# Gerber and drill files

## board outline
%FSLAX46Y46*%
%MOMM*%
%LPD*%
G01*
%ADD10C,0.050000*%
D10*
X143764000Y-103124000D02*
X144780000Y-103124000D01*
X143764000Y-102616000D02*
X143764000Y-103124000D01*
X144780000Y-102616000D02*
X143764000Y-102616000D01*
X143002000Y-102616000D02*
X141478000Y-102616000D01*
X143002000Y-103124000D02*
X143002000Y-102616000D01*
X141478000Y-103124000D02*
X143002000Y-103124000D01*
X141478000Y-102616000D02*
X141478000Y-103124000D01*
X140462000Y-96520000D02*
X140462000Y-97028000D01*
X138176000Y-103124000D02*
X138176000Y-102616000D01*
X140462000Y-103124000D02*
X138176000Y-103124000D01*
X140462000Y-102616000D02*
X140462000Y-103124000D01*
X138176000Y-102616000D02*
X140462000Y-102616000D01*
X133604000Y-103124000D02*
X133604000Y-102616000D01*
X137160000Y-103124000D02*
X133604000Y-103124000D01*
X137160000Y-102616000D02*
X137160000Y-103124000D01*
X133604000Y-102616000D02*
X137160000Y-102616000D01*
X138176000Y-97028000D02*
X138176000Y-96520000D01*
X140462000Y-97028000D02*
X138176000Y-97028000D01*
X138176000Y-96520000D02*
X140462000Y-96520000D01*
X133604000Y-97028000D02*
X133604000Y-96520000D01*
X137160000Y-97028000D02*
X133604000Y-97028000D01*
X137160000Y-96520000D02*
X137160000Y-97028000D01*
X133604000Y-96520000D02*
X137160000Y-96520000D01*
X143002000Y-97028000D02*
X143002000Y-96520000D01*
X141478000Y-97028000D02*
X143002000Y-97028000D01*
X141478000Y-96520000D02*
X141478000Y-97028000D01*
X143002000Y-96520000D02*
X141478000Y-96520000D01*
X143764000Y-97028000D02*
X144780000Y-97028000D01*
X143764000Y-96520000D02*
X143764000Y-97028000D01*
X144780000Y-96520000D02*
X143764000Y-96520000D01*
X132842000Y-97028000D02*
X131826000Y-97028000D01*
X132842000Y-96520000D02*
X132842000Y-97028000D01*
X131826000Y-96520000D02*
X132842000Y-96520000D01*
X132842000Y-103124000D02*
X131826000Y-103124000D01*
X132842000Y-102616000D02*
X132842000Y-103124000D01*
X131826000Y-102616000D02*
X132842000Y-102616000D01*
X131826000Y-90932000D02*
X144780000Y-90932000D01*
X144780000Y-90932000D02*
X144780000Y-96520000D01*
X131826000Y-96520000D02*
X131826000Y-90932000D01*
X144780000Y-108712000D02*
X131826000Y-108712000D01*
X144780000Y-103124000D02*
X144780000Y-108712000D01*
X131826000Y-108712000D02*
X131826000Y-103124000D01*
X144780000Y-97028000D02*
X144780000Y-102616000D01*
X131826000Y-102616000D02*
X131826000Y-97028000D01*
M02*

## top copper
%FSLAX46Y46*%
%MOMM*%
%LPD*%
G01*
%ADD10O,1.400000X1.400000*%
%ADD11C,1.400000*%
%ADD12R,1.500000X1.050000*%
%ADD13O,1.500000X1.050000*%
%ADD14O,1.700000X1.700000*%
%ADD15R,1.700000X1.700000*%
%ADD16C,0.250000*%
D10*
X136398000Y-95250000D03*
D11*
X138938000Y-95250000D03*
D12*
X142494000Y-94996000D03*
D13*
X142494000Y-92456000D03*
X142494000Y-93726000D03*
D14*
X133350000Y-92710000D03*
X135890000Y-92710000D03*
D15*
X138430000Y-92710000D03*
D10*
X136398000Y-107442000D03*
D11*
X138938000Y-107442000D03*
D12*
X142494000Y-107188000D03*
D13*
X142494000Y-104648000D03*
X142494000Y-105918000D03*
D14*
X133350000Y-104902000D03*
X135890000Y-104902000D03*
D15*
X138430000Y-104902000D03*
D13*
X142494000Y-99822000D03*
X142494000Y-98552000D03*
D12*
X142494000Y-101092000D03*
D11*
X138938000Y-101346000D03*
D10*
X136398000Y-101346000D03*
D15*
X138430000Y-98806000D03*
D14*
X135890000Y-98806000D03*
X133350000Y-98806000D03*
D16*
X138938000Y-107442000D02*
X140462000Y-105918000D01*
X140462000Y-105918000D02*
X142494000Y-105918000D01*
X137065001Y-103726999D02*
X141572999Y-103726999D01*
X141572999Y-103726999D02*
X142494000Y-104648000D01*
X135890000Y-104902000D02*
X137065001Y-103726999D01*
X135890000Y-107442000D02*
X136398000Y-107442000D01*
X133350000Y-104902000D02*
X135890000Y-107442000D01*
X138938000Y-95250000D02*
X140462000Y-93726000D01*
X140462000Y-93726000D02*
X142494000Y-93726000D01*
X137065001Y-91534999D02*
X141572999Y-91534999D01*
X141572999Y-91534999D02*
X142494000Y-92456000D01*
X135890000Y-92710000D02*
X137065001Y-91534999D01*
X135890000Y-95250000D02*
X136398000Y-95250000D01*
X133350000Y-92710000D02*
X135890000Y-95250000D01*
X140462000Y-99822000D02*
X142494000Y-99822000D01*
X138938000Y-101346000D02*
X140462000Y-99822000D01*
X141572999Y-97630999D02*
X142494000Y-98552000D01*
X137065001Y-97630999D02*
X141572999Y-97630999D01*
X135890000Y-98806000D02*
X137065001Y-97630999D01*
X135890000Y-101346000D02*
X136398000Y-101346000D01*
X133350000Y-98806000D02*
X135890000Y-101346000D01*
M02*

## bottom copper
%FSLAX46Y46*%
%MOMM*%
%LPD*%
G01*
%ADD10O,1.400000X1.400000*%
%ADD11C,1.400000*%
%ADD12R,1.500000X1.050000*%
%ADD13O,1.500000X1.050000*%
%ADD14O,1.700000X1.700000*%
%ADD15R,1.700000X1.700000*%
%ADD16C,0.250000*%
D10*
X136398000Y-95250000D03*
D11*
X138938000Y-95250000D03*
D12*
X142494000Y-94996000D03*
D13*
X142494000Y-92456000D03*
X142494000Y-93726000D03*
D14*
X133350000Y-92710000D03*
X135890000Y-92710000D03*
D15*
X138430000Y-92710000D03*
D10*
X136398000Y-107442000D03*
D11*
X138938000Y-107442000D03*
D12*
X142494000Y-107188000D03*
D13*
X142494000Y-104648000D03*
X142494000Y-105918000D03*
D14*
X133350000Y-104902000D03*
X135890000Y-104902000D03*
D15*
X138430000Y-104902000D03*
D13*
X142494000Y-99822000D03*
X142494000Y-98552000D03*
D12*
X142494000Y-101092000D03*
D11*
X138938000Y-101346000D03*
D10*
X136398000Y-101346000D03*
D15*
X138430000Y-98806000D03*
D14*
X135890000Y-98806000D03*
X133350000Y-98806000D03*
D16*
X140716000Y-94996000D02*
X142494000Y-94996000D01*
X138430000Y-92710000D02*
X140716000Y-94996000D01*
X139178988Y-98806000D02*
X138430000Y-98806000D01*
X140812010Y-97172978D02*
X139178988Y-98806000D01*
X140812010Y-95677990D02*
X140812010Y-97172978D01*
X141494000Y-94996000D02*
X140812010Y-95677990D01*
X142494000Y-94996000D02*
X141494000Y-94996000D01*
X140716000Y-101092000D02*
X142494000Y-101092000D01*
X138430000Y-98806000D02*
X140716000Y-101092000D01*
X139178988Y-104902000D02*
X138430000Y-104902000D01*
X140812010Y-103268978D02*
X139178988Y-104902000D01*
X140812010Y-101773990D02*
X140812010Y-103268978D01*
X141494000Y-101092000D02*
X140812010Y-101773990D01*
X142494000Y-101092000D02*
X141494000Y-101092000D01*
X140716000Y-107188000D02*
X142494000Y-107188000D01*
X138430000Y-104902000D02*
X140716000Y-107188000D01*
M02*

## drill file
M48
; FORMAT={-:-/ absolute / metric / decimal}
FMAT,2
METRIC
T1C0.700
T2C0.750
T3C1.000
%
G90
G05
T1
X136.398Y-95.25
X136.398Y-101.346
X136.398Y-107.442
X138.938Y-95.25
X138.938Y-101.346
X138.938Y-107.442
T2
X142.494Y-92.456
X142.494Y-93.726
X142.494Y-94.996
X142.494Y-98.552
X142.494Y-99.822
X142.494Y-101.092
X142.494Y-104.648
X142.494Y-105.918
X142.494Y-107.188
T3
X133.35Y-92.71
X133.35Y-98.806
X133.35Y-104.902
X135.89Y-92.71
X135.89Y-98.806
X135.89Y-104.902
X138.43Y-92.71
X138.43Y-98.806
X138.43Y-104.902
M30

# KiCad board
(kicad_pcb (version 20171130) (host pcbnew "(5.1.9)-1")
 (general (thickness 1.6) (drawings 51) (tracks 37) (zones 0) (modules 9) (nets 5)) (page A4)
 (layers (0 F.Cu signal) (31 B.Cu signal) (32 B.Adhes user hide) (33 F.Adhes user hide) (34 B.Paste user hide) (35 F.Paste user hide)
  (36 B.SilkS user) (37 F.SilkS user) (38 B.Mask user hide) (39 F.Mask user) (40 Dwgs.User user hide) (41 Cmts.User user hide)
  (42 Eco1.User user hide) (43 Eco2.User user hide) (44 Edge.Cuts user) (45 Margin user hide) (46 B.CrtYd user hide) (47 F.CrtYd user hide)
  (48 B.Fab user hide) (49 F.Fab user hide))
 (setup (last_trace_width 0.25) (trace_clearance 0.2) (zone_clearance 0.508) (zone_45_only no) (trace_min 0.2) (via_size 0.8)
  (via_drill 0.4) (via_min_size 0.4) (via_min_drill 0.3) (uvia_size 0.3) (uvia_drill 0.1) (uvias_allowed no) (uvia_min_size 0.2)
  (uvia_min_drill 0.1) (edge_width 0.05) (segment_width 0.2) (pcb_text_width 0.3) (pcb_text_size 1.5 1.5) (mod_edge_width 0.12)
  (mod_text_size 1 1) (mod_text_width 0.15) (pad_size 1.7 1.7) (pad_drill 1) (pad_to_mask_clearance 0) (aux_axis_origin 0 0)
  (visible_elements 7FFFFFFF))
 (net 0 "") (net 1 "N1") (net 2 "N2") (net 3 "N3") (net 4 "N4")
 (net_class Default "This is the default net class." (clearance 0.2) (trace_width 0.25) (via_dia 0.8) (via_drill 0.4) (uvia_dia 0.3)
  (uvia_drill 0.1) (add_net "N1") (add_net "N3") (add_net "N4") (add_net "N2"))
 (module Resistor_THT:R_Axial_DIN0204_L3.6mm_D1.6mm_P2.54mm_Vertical (layer F.Cu) (at 138.938 95.25 180)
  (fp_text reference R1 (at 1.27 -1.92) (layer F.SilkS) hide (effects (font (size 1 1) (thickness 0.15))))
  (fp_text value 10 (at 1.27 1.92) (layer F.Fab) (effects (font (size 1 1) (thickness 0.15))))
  (pad 2 thru_hole oval (at 2.54 0 180) (size 1.4 1.4) (drill 0.7) (layers *.Cu *.Mask))
  (pad 1 thru_hole circle (at 0 0 180) (size 1.4 1.4) (drill 0.7) (layers *.Cu *.Mask)))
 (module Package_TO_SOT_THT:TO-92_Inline (layer F.Cu) (at 142.494 94.996 90)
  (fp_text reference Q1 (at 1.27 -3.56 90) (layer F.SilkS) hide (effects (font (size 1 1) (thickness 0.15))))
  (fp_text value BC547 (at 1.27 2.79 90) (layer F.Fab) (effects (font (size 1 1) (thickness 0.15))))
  (pad 1 thru_hole rect (at 0 0 90) (size 1.05 1.5) (drill 0.75) (layers *.Cu *.Mask) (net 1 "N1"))
  (pad 3 thru_hole oval (at 2.54 0 90) (size 1.05 1.5) (drill 0.75) (layers *.Cu *.Mask))
  (pad 2 thru_hole oval (at 1.27 0 90) (size 1.05 1.5) (drill 0.75) (layers *.Cu *.Mask)))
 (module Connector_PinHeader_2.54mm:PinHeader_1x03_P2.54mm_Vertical (layer F.Cu) (at 138.43 92.71 270)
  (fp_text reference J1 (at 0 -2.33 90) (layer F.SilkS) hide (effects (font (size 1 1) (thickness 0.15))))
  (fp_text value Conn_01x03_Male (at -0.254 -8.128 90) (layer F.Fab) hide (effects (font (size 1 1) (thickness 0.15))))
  (pad 3 thru_hole oval (at 0 5.08 270) (size 1.7 1.7) (drill 1) (layers *.Cu *.Mask))
  (pad 2 thru_hole oval (at 0 2.54 270) (size 1.7 1.7) (drill 1) (layers *.Cu *.Mask))
  (pad 1 thru_hole rect (at 0 0 270) (size 1.7 1.7) (drill 1) (layers *.Cu *.Mask) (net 1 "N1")))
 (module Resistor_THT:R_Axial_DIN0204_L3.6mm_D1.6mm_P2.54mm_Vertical (layer F.Cu) (at 138.938 107.442 180)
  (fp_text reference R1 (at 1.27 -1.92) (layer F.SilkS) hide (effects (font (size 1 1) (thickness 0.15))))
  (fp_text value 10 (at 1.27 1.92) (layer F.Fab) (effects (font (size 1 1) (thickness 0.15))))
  (pad 2 thru_hole oval (at 2.54 0 180) (size 1.4 1.4) (drill 0.7) (layers *.Cu *.Mask))
  (pad 1 thru_hole circle (at 0 0 180) (size 1.4 1.4) (drill 0.7) (layers *.Cu *.Mask)))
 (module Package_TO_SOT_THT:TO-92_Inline (layer F.Cu) (at 142.494 107.188 90)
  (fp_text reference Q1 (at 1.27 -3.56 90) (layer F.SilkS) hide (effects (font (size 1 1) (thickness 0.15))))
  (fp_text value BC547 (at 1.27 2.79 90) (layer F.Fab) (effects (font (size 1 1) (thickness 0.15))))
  (pad 1 thru_hole rect (at 0 0 90) (size 1.05 1.5) (drill 0.75) (layers *.Cu *.Mask) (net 1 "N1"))
  (pad 3 thru_hole oval (at 2.54 0 90) (size 1.05 1.5) (drill 0.75) (layers *.Cu *.Mask))
  (pad 2 thru_hole oval (at 1.27 0 90) (size 1.05 1.5) (drill 0.75) (layers *.Cu *.Mask)))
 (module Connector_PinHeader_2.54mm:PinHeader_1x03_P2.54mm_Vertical (layer F.Cu) (at 138.43 104.902 270)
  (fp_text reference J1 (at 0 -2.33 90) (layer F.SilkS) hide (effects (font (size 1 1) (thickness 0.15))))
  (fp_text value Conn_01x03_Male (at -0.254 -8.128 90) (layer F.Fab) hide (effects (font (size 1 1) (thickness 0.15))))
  (pad 3 thru_hole oval (at 0 5.08 270) (size 1.7 1.7) (drill 1) (layers *.Cu *.Mask))
  (pad 2 thru_hole oval (at 0 2.54 270) (size 1.7 1.7) (drill 1) (layers *.Cu *.Mask))
  (pad 1 thru_hole rect (at 0 0 270) (size 1.7 1.7) (drill 1) (layers *.Cu *.Mask) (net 1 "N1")))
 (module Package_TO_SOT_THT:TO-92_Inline (layer F.Cu) (at 142.494 101.092 90)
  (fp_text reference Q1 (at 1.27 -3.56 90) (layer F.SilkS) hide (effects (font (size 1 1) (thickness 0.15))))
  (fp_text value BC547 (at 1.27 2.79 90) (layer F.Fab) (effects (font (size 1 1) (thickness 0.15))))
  (pad 2 thru_hole oval (at 1.27 0 90) (size 1.05 1.5) (drill 0.75) (layers *.Cu *.Mask) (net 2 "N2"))
  (pad 3 thru_hole oval (at 2.54 0 90) (size 1.05 1.5) (drill 0.75) (layers *.Cu *.Mask) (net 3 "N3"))
  (pad 1 thru_hole rect (at 0 0 90) (size 1.05 1.5) (drill 0.75) (layers *.Cu *.Mask) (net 1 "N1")))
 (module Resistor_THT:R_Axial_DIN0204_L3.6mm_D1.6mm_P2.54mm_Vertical (layer F.Cu) (at 138.938 101.346 180)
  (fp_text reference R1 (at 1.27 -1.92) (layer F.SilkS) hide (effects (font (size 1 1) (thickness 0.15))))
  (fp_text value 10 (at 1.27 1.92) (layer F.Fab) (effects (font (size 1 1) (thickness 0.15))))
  (pad 1 thru_hole circle (at 0 0 180) (size 1.4 1.4) (drill 0.7) (layers *.Cu *.Mask) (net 2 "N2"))
  (pad 2 thru_hole oval (at 2.54 0 180) (size 1.4 1.4) (drill 0.7) (layers *.Cu *.Mask) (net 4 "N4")))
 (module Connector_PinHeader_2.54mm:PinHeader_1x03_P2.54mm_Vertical (layer F.Cu) (at 138.43 98.806 270)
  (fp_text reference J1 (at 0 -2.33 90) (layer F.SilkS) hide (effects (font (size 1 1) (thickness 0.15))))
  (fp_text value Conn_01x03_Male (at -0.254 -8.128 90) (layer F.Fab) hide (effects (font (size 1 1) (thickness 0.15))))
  (pad 1 thru_hole rect (at 0 0 270) (size 1.7 1.7) (drill 1) (layers *.Cu *.Mask) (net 1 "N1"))
  (pad 2 thru_hole oval (at 0 2.54 270) (size 1.7 1.7) (drill 1) (layers *.Cu *.Mask) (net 3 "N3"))
  (pad 3 thru_hole oval (at 0 5.08 270) (size 1.7 1.7) (drill 1) (layers *.Cu *.Mask) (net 4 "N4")))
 (gr_line (start 143.764 103.124) (end 144.78 103.124) (layer Edge.Cuts) (width 0.05))
 (gr_line (start 143.764 102.616) (end 143.764 103.124) (layer Edge.Cuts) (width 0.05))
 (gr_line (start 144.78 102.616) (end 143.764 102.616) (layer Edge.Cuts) (width 0.05))
 (gr_line (start 143.002 102.616) (end 141.478 102.616) (layer Edge.Cuts) (width 0.05))
 (gr_line (start 143.002 103.124) (end 143.002 102.616) (layer Edge.Cuts) (width 0.05))
 (gr_line (start 141.478 103.124) (end 143.002 103.124) (layer Edge.Cuts) (width 0.05))
 (gr_line (start 141.478 102.616) (end 141.478 103.124) (layer Edge.Cuts) (width 0.05))
 (gr_line (start 140.462 96.52) (end 140.462 97.028) (layer Edge.Cuts) (width 0.05))
 (gr_line (start 138.176 103.124) (end 138.176 102.616) (layer Edge.Cuts) (width 0.05))
 (gr_line (start 140.462 103.124) (end 138.176 103.124) (layer Edge.Cuts) (width 0.05))
 (gr_line (start 140.462 102.616) (end 140.462 103.124) (layer Edge.Cuts) (width 0.05))
 (gr_line (start 138.176 102.616) (end 140.462 102.616) (layer Edge.Cuts) (width 0.05))
 (gr_line (start 133.604 103.124) (end 133.604 102.616) (layer Edge.Cuts) (width 0.05))
 (gr_line (start 137.16 103.124) (end 133.604 103.124) (layer Edge.Cuts) (width 0.05))
 (gr_line (start 137.16 102.616) (end 137.16 103.124) (layer Edge.Cuts) (width 0.05))
 (gr_line (start 133.604 102.616) (end 137.16 102.616) (layer Edge.Cuts) (width 0.05))
 (gr_line (start 138.176 97.028) (end 138.176 96.52) (layer Edge.Cuts) (width 0.05))
 (gr_line (start 140.462 97.028) (end 138.176 97.028) (layer Edge.Cuts) (width 0.05))
 (gr_line (start 138.176 96.52) (end 140.462 96.52) (layer Edge.Cuts) (width 0.05))
 (gr_line (start 133.604 97.028) (end 133.604 96.52) (layer Edge.Cuts) (width 0.05))
 (gr_line (start 137.16 97.028) (end 133.604 97.028) (layer Edge.Cuts) (width 0.05))
 (gr_line (start 137.16 96.52) (end 137.16 97.028) (layer Edge.Cuts) (width 0.05))
 (gr_line (start 133.604 96.52) (end 137.16 96.52) (layer Edge.Cuts) (width 0.05))
 (gr_line (start 143.002 97.028) (end 143.002 96.52) (layer Edge.Cuts) (width 0.05))
 (gr_line (start 141.478 97.028) (end 143.002 97.028) (layer Edge.Cuts) (width 0.05))
 (gr_line (start 141.478 96.52) (end 141.478 97.028) (layer Edge.Cuts) (width 0.05))
 (gr_line (start 143.002 96.52) (end 141.478 96.52) (layer Edge.Cuts) (width 0.05))
 (gr_line (start 143.764 97.028) (end 144.78 97.028) (layer Edge.Cuts) (width 0.05))
 (gr_line (start 143.764 96.52) (end 143.764 97.028) (layer Edge.Cuts) (width 0.05))
 (gr_line (start 144.78 96.52) (end 143.764 96.52) (layer Edge.Cuts) (width 0.05))
 (gr_line (start 132.842 97.028) (end 131.826 97.028) (layer Edge.Cuts) (width 0.05))
 (gr_line (start 132.842 96.52) (end 132.842 97.028) (layer Edge.Cuts) (width 0.05))
 (gr_line (start 131.826 96.52) (end 132.842 96.52) (layer Edge.Cuts) (width 0.05))
 (gr_line (start 132.842 103.124) (end 131.826 103.124) (layer Edge.Cuts) (width 0.05))
 (gr_line (start 132.842 102.616) (end 132.842 103.124) (layer Edge.Cuts) (width 0.05))
 (gr_line (start 131.826 102.616) (end 132.842 102.616) (layer Edge.Cuts) (width 0.05))
 (gr_line (start 131.826 90.932) (end 144.78 90.932) (layer Edge.Cuts) (width 0.05))
 (gr_line (start 144.78 90.932) (end 144.78 96.52) (layer Edge.Cuts) (width 0.05))
 (gr_line (start 131.826 96.52) (end 131.826 90.932) (layer Edge.Cuts) (width 0.05))
 (gr_line (start 144.78 108.712) (end 131.826 108.712) (layer Edge.Cuts) (width 0.05))
 (gr_line (start 144.78 103.124) (end 144.78 108.712) (layer Edge.Cuts) (width 0.05))
 (gr_line (start 131.826 108.712) (end 131.826 103.124) (layer Edge.Cuts) (width 0.05))
 (gr_line (start 144.78 97.028) (end 144.78 102.616) (layer Edge.Cuts) (width 0.05))
 (gr_line (start 131.826 102.616) (end 131.826 97.028) (layer Edge.Cuts) (width 0.05))
 (segment (start 138.938 107.442) (end 140.462 105.918) (width 0.25) (layer F.Cu) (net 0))
 (segment (start 140.462 105.918) (end 142.494 105.918) (width 0.25) (layer F.Cu) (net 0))
 (segment (start 137.065001 103.726999) (end 141.572999 103.726999) (width 0.25) (layer F.Cu) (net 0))
 (segment (start 141.572999 103.726999) (end 142.494 104.648) (width 0.25) (layer F.Cu) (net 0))
 (segment (start 135.89 104.902) (end 137.065001 103.726999) (width 0.25) (layer F.Cu) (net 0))
 (segment (start 135.89 107.442) (end 136.398 107.442) (width 0.25) (layer F.Cu) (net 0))
 (segment (start 133.35 104.902) (end 135.89 107.442) (width 0.25) (layer F.Cu) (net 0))
 (segment (start 138.938 95.25) (end 140.462 93.726) (width 0.25) (layer F.Cu) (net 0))
 (segment (start 140.462 93.726) (end 142.494 93.726) (width 0.25) (layer F.Cu) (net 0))
 (segment (start 137.065001 91.534999) (end 141.572999 91.534999) (width 0.25) (layer F.Cu) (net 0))
 (segment (start 141.572999 91.534999) (end 142.494 92.456) (width 0.25) (layer F.Cu) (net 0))
 (segment (start 135.89 92.71) (end 137.065001 91.534999) (width 0.25) (layer F.Cu) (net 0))
 (segment (start 135.89 95.25) (end 136.398 95.25) (width 0.25) (layer F.Cu) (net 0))
 (segment (start 133.35 92.71) (end 135.89 95.25) (width 0.25) (layer F.Cu) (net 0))
 (segment (start 140.716 94.996) (end 142.494 94.996) (width 0.25) (layer B.Cu) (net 1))
 (segment (start 138.43 92.71) (end 140.716 94.996) (width 0.25) (layer B.Cu) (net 1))
 (segment (start 139.178988 98.806) (end 138.43 98.806) (width 0.25) (layer B.Cu) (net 1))
 (segment (start 140.81201 97.172978) (end 139.178988 98.806) (width 0.25) (layer B.Cu) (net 1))
 (segment (start 140.81201 95.67799) (end 140.81201 97.172978) (width 0.25) (layer B.Cu) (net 1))
 (segment (start 141.494 94.996) (end 140.81201 95.67799) (width 0.25) (layer B.Cu) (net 1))
 (segment (start 142.494 94.996) (end 141.494 94.996) (width 0.25) (layer B.Cu) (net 1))
 (segment (start 140.716 101.092) (end 142.494 101.092) (width 0.25) (layer B.Cu) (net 1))
 (segment (start 138.43 98.806) (end 140.716 101.092) (width 0.25) (layer B.Cu) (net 1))
 (segment (start 139.178988 104.902) (end 138.43 104.902) (width 0.25) (layer B.Cu) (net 1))
 (segment (start 140.81201 103.268978) (end 139.178988 104.902) (width 0.25) (layer B.Cu) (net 1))
 (segment (start 140.81201 101.77399) (end 140.81201 103.268978) (width 0.25) (layer B.Cu) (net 1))
 (segment (start 141.494 101.092) (end 140.81201 101.77399) (width 0.25) (layer B.Cu) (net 1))
 (segment (start 142.494 101.092) (end 141.494 101.092) (width 0.25) (layer B.Cu) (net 1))
 (segment (start 140.716 107.188) (end 142.494 107.188) (width 0.25) (layer B.Cu) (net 1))
 (segment (start 138.43 104.902) (end 140.716 107.188) (width 0.25) (layer B.Cu) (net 1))
 (segment (start 140.462 99.822) (end 142.494 99.822) (width 0.25) (layer F.Cu) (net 2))
 (segment (start 138.938 101.346) (end 140.462 99.822) (width 0.25) (layer F.Cu) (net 2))
 (segment (start 141.572999 97.630999) (end 142.494 98.552) (width 0.25) (layer F.Cu) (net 3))
 (segment (start 137.065001 97.630999) (end 141.572999 97.630999) (width 0.25) (layer F.Cu) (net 3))
 (segment (start 135.89 98.806) (end 137.065001 97.630999) (width 0.25) (layer F.Cu) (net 3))
 (segment (start 135.89 101.346) (end 136.398 101.346) (width 0.25) (layer F.Cu) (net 4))
 (segment (start 133.35 98.806) (end 135.89 101.346) (width 0.25) (layer F.Cu) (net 4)))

